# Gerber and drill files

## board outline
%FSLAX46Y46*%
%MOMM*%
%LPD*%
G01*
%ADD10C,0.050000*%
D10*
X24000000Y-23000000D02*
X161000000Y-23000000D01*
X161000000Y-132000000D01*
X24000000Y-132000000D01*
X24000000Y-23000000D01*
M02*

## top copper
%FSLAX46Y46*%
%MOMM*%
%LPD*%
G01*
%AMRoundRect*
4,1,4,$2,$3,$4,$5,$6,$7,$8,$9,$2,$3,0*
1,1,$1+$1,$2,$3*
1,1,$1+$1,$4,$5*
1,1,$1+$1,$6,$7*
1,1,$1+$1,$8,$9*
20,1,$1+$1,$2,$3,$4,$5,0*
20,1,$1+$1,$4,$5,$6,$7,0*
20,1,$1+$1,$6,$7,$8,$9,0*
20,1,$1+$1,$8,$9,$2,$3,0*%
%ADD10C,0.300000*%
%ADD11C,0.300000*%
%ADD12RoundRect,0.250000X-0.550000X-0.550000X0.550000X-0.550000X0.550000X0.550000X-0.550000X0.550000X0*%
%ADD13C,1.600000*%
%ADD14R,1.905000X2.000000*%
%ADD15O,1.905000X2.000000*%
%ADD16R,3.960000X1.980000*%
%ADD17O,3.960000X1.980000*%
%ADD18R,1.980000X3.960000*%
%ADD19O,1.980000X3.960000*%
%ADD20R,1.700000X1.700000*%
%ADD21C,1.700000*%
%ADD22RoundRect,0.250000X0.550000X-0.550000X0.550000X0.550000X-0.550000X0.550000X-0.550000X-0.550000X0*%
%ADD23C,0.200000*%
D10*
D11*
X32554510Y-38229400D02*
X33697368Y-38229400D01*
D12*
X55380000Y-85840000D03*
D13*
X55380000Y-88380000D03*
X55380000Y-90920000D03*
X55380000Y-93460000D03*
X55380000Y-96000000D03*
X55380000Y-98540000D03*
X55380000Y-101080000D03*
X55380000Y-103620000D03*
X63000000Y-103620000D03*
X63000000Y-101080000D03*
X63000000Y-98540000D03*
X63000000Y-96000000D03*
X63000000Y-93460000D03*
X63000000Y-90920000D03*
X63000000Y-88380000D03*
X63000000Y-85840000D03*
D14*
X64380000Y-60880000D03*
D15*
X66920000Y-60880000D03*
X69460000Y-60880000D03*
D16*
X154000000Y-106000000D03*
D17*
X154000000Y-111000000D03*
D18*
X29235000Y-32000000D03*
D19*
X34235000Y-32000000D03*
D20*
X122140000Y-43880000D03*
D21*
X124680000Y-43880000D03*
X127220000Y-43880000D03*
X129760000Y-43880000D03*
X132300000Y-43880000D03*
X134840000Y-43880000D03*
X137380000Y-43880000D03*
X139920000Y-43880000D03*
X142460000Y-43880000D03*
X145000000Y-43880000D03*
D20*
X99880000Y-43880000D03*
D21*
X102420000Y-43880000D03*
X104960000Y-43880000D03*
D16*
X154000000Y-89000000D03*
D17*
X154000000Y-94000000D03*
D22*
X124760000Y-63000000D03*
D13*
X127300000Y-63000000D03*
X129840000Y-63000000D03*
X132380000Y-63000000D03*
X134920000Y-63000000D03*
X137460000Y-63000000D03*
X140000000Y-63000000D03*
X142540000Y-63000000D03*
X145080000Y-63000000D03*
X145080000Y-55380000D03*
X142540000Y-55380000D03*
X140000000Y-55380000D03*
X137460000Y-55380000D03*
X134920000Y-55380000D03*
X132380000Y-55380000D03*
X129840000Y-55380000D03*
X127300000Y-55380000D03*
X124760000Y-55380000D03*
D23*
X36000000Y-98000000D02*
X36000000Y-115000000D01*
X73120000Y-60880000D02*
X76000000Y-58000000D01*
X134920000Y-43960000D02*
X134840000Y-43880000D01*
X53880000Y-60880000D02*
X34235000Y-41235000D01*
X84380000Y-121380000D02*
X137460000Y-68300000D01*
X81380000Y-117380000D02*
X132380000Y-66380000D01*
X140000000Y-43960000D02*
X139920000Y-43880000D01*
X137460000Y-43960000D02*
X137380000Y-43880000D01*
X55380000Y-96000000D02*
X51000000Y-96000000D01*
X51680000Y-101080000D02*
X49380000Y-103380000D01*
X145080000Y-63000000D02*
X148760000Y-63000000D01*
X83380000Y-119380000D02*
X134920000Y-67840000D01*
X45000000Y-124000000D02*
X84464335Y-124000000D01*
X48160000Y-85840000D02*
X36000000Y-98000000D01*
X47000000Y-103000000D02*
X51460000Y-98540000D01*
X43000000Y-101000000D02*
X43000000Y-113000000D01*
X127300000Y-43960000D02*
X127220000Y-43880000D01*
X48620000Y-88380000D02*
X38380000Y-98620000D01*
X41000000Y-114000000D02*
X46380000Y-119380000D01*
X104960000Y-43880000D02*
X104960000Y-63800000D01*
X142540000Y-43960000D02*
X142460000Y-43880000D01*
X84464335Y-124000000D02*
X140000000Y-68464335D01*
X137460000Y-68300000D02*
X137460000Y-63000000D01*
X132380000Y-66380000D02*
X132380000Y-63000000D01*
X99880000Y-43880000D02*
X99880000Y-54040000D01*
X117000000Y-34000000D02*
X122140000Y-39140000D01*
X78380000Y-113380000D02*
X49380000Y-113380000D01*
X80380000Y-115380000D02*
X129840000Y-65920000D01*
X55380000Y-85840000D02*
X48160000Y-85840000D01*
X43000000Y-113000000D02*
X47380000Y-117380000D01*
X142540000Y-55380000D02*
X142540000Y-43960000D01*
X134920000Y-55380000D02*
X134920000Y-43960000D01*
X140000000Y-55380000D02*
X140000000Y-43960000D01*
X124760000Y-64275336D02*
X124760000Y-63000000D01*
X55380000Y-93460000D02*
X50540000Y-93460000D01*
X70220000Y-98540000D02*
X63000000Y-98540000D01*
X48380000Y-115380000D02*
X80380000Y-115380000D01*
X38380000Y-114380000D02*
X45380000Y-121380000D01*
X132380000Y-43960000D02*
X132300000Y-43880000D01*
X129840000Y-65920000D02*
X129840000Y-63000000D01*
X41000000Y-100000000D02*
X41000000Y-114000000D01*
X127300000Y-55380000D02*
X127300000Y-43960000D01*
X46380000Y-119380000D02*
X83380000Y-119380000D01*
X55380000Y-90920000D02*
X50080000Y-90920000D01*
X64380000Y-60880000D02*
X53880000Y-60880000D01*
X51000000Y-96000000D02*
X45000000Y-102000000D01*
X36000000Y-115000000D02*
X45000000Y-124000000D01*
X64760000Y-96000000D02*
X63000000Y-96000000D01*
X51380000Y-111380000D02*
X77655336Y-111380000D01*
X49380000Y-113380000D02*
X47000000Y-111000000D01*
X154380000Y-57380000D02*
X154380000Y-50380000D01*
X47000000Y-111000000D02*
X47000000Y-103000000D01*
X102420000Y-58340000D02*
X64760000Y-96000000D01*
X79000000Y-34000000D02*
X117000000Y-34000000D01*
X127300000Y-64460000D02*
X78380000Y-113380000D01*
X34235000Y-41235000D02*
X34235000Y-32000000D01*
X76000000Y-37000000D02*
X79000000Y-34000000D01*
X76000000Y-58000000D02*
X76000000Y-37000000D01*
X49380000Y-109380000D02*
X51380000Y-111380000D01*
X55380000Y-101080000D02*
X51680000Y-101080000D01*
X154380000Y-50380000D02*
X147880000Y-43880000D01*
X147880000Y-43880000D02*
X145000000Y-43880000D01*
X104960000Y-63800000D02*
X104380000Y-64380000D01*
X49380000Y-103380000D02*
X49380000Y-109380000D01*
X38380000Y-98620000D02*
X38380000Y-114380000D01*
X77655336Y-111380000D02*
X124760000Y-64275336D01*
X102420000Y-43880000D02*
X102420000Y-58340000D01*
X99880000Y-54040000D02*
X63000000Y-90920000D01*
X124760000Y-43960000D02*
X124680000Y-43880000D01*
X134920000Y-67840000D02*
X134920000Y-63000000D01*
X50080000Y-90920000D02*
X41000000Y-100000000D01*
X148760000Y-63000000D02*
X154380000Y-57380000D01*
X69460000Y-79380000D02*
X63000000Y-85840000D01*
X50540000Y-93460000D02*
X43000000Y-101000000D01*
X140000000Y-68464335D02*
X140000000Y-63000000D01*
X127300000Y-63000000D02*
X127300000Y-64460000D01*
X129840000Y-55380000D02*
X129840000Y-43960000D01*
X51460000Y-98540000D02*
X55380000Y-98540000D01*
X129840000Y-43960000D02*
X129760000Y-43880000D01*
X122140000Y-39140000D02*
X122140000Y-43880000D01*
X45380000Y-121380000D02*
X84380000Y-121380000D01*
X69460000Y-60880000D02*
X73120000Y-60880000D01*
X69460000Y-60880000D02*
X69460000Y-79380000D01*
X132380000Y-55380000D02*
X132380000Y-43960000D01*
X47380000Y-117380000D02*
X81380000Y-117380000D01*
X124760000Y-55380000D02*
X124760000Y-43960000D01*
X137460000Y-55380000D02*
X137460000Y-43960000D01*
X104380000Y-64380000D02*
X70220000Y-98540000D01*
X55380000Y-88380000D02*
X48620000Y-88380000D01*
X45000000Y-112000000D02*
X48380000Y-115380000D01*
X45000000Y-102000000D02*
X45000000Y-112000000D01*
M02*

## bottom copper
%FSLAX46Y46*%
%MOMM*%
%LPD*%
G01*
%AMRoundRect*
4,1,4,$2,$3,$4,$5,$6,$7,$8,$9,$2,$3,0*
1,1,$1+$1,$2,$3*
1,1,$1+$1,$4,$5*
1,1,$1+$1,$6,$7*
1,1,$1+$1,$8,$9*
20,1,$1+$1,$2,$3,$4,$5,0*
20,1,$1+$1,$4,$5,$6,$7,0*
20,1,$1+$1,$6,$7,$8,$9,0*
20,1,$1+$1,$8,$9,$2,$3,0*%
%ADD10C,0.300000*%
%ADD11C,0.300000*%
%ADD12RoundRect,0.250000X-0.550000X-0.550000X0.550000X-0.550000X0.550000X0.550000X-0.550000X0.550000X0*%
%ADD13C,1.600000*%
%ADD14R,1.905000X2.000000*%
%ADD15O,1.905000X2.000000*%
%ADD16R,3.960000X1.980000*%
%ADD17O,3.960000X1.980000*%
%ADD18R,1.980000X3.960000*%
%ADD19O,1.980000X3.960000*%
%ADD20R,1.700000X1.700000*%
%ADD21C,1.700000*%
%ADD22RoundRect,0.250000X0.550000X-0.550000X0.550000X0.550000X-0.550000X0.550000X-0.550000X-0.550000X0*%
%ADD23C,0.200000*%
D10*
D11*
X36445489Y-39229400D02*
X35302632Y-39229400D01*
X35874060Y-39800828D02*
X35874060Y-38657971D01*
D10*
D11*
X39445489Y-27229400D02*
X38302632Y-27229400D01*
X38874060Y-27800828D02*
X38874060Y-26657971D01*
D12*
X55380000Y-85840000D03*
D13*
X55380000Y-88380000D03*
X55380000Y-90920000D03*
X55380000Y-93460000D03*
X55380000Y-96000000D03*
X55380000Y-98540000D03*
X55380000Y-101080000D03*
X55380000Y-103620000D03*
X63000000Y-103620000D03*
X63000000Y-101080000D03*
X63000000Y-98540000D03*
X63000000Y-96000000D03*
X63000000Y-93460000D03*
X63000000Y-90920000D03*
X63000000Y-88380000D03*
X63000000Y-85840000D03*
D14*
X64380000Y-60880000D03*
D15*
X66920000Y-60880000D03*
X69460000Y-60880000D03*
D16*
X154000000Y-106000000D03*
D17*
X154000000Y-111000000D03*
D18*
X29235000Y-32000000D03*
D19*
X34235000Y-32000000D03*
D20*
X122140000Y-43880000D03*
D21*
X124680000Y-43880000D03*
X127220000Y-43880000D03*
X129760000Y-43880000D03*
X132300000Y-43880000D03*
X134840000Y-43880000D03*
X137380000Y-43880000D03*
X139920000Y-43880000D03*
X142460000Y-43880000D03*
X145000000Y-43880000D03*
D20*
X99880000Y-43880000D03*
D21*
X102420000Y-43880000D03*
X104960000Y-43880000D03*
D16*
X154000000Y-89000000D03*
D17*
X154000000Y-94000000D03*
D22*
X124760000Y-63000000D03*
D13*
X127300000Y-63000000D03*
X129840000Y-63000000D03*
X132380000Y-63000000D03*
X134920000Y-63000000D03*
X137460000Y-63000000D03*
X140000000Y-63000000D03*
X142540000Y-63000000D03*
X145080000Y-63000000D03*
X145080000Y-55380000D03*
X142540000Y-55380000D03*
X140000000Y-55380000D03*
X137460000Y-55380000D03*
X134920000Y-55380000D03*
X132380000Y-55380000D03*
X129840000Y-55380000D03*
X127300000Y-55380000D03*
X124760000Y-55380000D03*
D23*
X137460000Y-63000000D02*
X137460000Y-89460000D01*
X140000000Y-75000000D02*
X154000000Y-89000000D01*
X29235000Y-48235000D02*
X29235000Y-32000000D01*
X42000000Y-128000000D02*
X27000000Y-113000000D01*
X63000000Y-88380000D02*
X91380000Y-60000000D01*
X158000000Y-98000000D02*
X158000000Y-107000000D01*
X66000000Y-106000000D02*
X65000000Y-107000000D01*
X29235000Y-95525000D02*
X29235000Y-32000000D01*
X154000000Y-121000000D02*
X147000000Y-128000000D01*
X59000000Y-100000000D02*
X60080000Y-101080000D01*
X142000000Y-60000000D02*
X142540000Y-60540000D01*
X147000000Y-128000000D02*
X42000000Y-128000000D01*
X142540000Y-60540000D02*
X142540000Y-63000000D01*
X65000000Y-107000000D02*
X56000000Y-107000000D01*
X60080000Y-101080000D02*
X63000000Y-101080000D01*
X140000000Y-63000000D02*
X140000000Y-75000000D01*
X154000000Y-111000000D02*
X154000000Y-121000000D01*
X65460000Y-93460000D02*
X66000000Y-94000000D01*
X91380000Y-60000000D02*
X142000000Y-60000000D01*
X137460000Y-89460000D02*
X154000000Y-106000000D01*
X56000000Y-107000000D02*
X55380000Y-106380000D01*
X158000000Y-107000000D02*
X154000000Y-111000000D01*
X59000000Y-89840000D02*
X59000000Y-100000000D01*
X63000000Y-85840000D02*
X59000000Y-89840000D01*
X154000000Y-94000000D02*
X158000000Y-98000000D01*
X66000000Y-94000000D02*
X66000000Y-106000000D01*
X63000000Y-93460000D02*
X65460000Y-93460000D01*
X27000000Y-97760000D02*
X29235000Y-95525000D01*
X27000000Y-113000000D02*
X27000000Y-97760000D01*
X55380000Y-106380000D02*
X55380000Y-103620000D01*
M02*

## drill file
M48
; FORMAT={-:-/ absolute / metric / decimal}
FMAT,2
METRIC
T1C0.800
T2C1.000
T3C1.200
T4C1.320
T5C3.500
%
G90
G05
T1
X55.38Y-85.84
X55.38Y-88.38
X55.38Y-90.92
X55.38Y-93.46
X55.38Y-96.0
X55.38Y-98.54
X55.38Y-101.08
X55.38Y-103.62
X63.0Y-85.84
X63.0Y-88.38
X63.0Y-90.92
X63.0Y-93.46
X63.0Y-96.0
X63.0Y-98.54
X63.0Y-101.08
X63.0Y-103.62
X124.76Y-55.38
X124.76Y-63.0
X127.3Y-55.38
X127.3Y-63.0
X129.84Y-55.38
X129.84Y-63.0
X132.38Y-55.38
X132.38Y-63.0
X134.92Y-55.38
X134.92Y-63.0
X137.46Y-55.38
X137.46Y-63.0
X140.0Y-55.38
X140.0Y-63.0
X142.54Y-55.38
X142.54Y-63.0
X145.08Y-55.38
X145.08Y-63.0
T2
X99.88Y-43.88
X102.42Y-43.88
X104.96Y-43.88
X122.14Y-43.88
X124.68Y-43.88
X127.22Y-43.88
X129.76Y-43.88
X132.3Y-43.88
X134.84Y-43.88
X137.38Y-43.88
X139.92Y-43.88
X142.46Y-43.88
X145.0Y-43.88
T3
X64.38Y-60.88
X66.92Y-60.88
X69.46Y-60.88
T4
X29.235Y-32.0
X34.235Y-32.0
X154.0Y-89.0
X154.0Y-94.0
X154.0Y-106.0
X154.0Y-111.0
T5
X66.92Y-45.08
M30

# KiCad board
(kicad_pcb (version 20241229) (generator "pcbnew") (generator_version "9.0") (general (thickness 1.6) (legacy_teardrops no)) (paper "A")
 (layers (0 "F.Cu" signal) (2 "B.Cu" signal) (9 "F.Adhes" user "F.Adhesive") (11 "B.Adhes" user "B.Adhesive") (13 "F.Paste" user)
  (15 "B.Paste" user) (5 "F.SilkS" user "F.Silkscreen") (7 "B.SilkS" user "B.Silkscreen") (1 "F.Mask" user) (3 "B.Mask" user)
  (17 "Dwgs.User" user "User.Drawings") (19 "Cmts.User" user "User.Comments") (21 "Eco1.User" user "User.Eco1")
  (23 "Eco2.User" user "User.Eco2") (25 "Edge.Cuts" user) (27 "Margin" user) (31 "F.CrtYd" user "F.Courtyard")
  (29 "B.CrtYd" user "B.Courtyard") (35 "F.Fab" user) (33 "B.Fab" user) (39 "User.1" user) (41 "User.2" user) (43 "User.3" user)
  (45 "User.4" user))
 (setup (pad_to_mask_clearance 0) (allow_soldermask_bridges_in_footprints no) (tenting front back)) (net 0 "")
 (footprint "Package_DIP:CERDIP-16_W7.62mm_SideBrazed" (layer "F.Cu") (at 55.38 85.84)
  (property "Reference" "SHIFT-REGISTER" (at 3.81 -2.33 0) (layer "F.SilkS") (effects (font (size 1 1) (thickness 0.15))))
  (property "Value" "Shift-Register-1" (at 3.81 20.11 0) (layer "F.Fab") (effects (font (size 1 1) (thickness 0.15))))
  (pad "1" thru_hole roundrect (at 0 0) (size 1.6 1.6) (drill 0.8) (layers "*.Cu" "*.Mask") (remove_unused_layers no)
   (roundrect_rratio 0.15625))
  (pad "2" thru_hole circle (at 0 2.54) (size 1.6 1.6) (drill 0.8) (layers "*.Cu" "*.Mask") (remove_unused_layers no))
  (pad "3" thru_hole circle (at 0 5.08) (size 1.6 1.6) (drill 0.8) (layers "*.Cu" "*.Mask") (remove_unused_layers no))
  (pad "4" thru_hole circle (at 0 7.62) (size 1.6 1.6) (drill 0.8) (layers "*.Cu" "*.Mask") (remove_unused_layers no))
  (pad "5" thru_hole circle (at 0 10.16) (size 1.6 1.6) (drill 0.8) (layers "*.Cu" "*.Mask") (remove_unused_layers no))
  (pad "6" thru_hole circle (at 0 12.7) (size 1.6 1.6) (drill 0.8) (layers "*.Cu" "*.Mask") (remove_unused_layers no))
  (pad "7" thru_hole circle (at 0 15.24) (size 1.6 1.6) (drill 0.8) (layers "*.Cu" "*.Mask") (remove_unused_layers no))
  (pad "8" thru_hole circle (at 0 17.78) (size 1.6 1.6) (drill 0.8) (layers "*.Cu" "*.Mask") (remove_unused_layers no))
  (pad "9" thru_hole circle (at 7.62 17.78) (size 1.6 1.6) (drill 0.8) (layers "*.Cu" "*.Mask") (remove_unused_layers no))
  (pad "10" thru_hole circle (at 7.62 15.24) (size 1.6 1.6) (drill 0.8) (layers "*.Cu" "*.Mask") (remove_unused_layers no))
  (pad "11" thru_hole circle (at 7.62 12.7) (size 1.6 1.6) (drill 0.8) (layers "*.Cu" "*.Mask") (remove_unused_layers no))
  (pad "12" thru_hole circle (at 7.62 10.16) (size 1.6 1.6) (drill 0.8) (layers "*.Cu" "*.Mask") (remove_unused_layers no))
  (pad "13" thru_hole circle (at 7.62 7.62) (size 1.6 1.6) (drill 0.8) (layers "*.Cu" "*.Mask") (remove_unused_layers no))
  (pad "14" thru_hole circle (at 7.62 5.08) (size 1.6 1.6) (drill 0.8) (layers "*.Cu" "*.Mask") (remove_unused_layers no))
  (pad "15" thru_hole circle (at 7.62 2.54) (size 1.6 1.6) (drill 0.8) (layers "*.Cu" "*.Mask") (remove_unused_layers no))
  (pad "16" thru_hole circle (at 7.62 0) (size 1.6 1.6) (drill 0.8) (layers "*.Cu" "*.Mask") (remove_unused_layers no)))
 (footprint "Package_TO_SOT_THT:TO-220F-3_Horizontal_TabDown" (layer "F.Cu") (at 64.38 60.88)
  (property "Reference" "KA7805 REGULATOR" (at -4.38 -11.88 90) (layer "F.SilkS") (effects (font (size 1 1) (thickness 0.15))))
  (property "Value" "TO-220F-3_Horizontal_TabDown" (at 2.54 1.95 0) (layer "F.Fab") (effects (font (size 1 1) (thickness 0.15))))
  (pad "" np_thru_hole circle (at 2.54 -15.8) (size 3.5 3.5) (drill 3.5) (layers "*.Cu" "*.Mask"))
  (pad "1" thru_hole rect (at 0 0) (size 1.905 2) (drill 1.2) (layers "*.Cu" "*.Mask") (remove_unused_layers no))
  (pad "2" thru_hole oval (at 2.54 0) (size 1.905 2) (drill 1.2) (layers "*.Cu" "*.Mask") (remove_unused_layers no))
  (pad "3" thru_hole oval (at 5.08 0) (size 1.905 2) (drill 1.2) (layers "*.Cu" "*.Mask") (remove_unused_layers no)))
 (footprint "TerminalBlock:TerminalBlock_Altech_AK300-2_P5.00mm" (layer "F.Cu") (at 154 106 -90)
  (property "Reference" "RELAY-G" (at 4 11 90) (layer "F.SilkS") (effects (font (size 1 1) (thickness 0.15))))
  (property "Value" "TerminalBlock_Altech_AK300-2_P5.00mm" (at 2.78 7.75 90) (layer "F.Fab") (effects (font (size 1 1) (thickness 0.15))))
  (pad "1" thru_hole rect (at 0 0 270) (size 1.98 3.96) (drill 1.32) (layers "*.Cu" "*.Mask") (remove_unused_layers no))
  (pad "2" thru_hole oval (at 5 0 270) (size 1.98 3.96) (drill 1.32) (layers "*.Cu" "*.Mask") (remove_unused_layers no)))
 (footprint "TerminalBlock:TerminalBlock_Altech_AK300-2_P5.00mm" (layer "F.Cu") (at 29.235 32)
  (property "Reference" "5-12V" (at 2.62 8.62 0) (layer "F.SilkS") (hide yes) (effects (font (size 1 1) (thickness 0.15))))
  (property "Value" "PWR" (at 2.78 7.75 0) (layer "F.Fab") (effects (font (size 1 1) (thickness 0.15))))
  (pad "1" thru_hole rect (at 0 0) (size 1.98 3.96) (drill 1.32) (layers "*.Cu" "*.Mask") (remove_unused_layers no))
  (pad "2" thru_hole oval (at 5 0) (size 1.98 3.96) (drill 1.32) (layers "*.Cu" "*.Mask") (remove_unused_layers no)))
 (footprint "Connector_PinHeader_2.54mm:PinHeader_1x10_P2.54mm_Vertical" (layer "F.Cu") (at 122.14 43.88 90)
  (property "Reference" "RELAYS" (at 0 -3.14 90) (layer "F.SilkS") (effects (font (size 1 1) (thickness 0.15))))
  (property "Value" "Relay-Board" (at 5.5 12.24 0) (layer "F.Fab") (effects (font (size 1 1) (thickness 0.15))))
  (pad "1" thru_hole rect (at 0 0 90) (size 1.7 1.7) (drill 1) (layers "*.Cu" "*.Mask") (remove_unused_layers no))
  (pad "2" thru_hole circle (at 0 2.54 90) (size 1.7 1.7) (drill 1) (layers "*.Cu" "*.Mask") (remove_unused_layers no))
  (pad "3" thru_hole circle (at 0 5.08 90) (size 1.7 1.7) (drill 1) (layers "*.Cu" "*.Mask") (remove_unused_layers no))
  (pad "4" thru_hole circle (at 0 7.62 90) (size 1.7 1.7) (drill 1) (layers "*.Cu" "*.Mask") (remove_unused_layers no))
  (pad "5" thru_hole circle (at 0 10.16 90) (size 1.7 1.7) (drill 1) (layers "*.Cu" "*.Mask") (remove_unused_layers no))
  (pad "6" thru_hole circle (at 0 12.7 90) (size 1.7 1.7) (drill 1) (layers "*.Cu" "*.Mask") (remove_unused_layers no))
  (pad "7" thru_hole circle (at 0 15.24 90) (size 1.7 1.7) (drill 1) (layers "*.Cu" "*.Mask") (remove_unused_layers no))
  (pad "8" thru_hole circle (at 0 17.78 90) (size 1.7 1.7) (drill 1) (layers "*.Cu" "*.Mask") (remove_unused_layers no))
  (pad "9" thru_hole circle (at 0 20.32 90) (size 1.7 1.7) (drill 1) (layers "*.Cu" "*.Mask") (remove_unused_layers no))
  (pad "10" thru_hole circle (at 0 22.86 90) (size 1.7 1.7) (drill 1) (layers "*.Cu" "*.Mask") (remove_unused_layers no)))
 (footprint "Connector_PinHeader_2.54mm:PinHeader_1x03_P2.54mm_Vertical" (layer "F.Cu") (at 99.88 43.88 90)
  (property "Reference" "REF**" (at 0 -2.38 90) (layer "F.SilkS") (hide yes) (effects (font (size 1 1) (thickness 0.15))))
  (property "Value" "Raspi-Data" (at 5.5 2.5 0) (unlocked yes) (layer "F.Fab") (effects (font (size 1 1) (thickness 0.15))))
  (pad "1" thru_hole rect (at 0 0 90) (size 1.7 1.7) (drill 1) (layers "*.Cu" "*.Mask") (remove_unused_layers no))
  (pad "2" thru_hole circle (at 0 2.54 90) (size 1.7 1.7) (drill 1) (layers "*.Cu" "*.Mask") (remove_unused_layers no))
  (pad "3" thru_hole circle (at 0 5.08 90) (size 1.7 1.7) (drill 1) (layers "*.Cu" "*.Mask") (remove_unused_layers no)))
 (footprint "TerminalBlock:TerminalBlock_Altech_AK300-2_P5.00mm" (layer "F.Cu") (at 154 89 -90)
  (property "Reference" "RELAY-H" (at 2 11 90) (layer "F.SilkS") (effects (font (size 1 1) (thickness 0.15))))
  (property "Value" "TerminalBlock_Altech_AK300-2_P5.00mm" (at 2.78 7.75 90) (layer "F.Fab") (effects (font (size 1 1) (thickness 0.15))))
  (pad "1" thru_hole rect (at 0 0 270) (size 1.98 3.96) (drill 1.32) (layers "*.Cu" "*.Mask") (remove_unused_layers no))
  (pad "2" thru_hole oval (at 5 0 270) (size 1.98 3.96) (drill 1.32) (layers "*.Cu" "*.Mask") (remove_unused_layers no)))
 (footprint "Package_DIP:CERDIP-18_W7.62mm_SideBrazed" (layer "F.Cu") (at 124.76 63 90)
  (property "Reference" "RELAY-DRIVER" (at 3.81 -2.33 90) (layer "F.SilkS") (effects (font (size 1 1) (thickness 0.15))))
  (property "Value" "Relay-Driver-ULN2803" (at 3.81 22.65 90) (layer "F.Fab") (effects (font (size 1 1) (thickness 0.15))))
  (pad "1" thru_hole roundrect (at 0 0 90) (size 1.6 1.6) (drill 0.8) (layers "*.Cu" "*.Mask") (remove_unused_layers no)
   (roundrect_rratio 0.15625))
  (pad "2" thru_hole circle (at 0 2.54 90) (size 1.6 1.6) (drill 0.8) (layers "*.Cu" "*.Mask") (remove_unused_layers no))
  (pad "3" thru_hole circle (at 0 5.08 90) (size 1.6 1.6) (drill 0.8) (layers "*.Cu" "*.Mask") (remove_unused_layers no))
  (pad "4" thru_hole circle (at 0 7.62 90) (size 1.6 1.6) (drill 0.8) (layers "*.Cu" "*.Mask") (remove_unused_layers no))
  (pad "5" thru_hole circle (at 0 10.16 90) (size 1.6 1.6) (drill 0.8) (layers "*.Cu" "*.Mask") (remove_unused_layers no))
  (pad "6" thru_hole circle (at 0 12.7 90) (size 1.6 1.6) (drill 0.8) (layers "*.Cu" "*.Mask") (remove_unused_layers no))
  (pad "7" thru_hole circle (at 0 15.24 90) (size 1.6 1.6) (drill 0.8) (layers "*.Cu" "*.Mask") (remove_unused_layers no))
  (pad "8" thru_hole circle (at 0 17.78 90) (size 1.6 1.6) (drill 0.8) (layers "*.Cu" "*.Mask") (remove_unused_layers no))
  (pad "9" thru_hole circle (at 0 20.32 90) (size 1.6 1.6) (drill 0.8) (layers "*.Cu" "*.Mask") (remove_unused_layers no))
  (pad "10" thru_hole circle (at 7.62 20.32 90) (size 1.6 1.6) (drill 0.8) (layers "*.Cu" "*.Mask") (remove_unused_layers no))
  (pad "11" thru_hole circle (at 7.62 17.78 90) (size 1.6 1.6) (drill 0.8) (layers "*.Cu" "*.Mask") (remove_unused_layers no))
  (pad "12" thru_hole circle (at 7.62 15.24 90) (size 1.6 1.6) (drill 0.8) (layers "*.Cu" "*.Mask") (remove_unused_layers no))
  (pad "13" thru_hole circle (at 7.62 12.7 90) (size 1.6 1.6) (drill 0.8) (layers "*.Cu" "*.Mask") (remove_unused_layers no))
  (pad "14" thru_hole circle (at 7.62 10.16 90) (size 1.6 1.6) (drill 0.8) (layers "*.Cu" "*.Mask") (remove_unused_layers no))
  (pad "15" thru_hole circle (at 7.62 7.62 90) (size 1.6 1.6) (drill 0.8) (layers "*.Cu" "*.Mask") (remove_unused_layers no))
  (pad "16" thru_hole circle (at 7.62 5.08 90) (size 1.6 1.6) (drill 0.8) (layers "*.Cu" "*.Mask") (remove_unused_layers no))
  (pad "17" thru_hole circle (at 7.62 2.54 90) (size 1.6 1.6) (drill 0.8) (layers "*.Cu" "*.Mask") (remove_unused_layers no))
  (pad "18" thru_hole circle (at 7.62 0 90) (size 1.6 1.6) (drill 0.8) (layers "*.Cu" "*.Mask") (remove_unused_layers no)))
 (gr_rect (start 24 23) (end 161 132) (stroke (width 0.05) (type default)) (fill no) (layer "Edge.Cuts"))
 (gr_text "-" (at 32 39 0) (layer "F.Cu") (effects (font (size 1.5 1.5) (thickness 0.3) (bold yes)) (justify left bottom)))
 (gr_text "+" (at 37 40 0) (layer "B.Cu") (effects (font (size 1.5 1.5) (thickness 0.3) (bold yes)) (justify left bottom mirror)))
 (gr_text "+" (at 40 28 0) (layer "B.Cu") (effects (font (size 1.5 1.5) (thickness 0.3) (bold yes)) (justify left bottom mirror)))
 (segment (start 36 98) (end 36 115) (width 0.2) (layer "F.Cu") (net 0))
 (segment (start 73.12 60.88) (end 76 58) (width 0.2) (layer "F.Cu") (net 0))
 (segment (start 134.92 43.96) (end 134.84 43.88) (width 0.2) (layer "F.Cu") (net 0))
 (segment (start 53.88 60.88) (end 34.235 41.235) (width 0.2) (layer "F.Cu") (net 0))
 (segment (start 84.38 121.38) (end 137.46 68.3) (width 0.2) (layer "F.Cu") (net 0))
 (segment (start 81.38 117.38) (end 132.38 66.38) (width 0.2) (layer "F.Cu") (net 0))
 (segment (start 140 43.96) (end 139.92 43.88) (width 0.2) (layer "F.Cu") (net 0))
 (segment (start 137.46 43.96) (end 137.38 43.88) (width 0.2) (layer "F.Cu") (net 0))
 (segment (start 55.38 96) (end 51 96) (width 0.2) (layer "F.Cu") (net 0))
 (segment (start 51.68 101.08) (end 49.38 103.38) (width 0.2) (layer "F.Cu") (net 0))
 (segment (start 145.08 63) (end 148.76 63) (width 0.2) (layer "F.Cu") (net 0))
 (segment (start 83.38 119.38) (end 134.92 67.84) (width 0.2) (layer "F.Cu") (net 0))
 (segment (start 45 124) (end 84.464335 124) (width 0.2) (layer "F.Cu") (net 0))
 (segment (start 48.16 85.84) (end 36 98) (width 0.2) (layer "F.Cu") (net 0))
 (segment (start 47 103) (end 51.46 98.54) (width 0.2) (layer "F.Cu") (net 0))
 (segment (start 43 101) (end 43 113) (width 0.2) (layer "F.Cu") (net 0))
 (segment (start 127.3 43.96) (end 127.22 43.88) (width 0.2) (layer "F.Cu") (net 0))
 (segment (start 48.62 88.38) (end 38.38 98.62) (width 0.2) (layer "F.Cu") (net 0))
 (segment (start 41 114) (end 46.38 119.38) (width 0.2) (layer "F.Cu") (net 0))
 (segment (start 104.96 43.88) (end 104.96 63.8) (width 0.2) (layer "F.Cu") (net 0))
 (segment (start 142.54 43.96) (end 142.46 43.88) (width 0.2) (layer "F.Cu") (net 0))
 (segment (start 84.464335 124) (end 140 68.464335) (width 0.2) (layer "F.Cu") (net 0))
 (segment (start 137.46 68.3) (end 137.46 63) (width 0.2) (layer "F.Cu") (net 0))
 (segment (start 132.38 66.38) (end 132.38 63) (width 0.2) (layer "F.Cu") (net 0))
 (segment (start 99.88 43.88) (end 99.88 54.04) (width 0.2) (layer "F.Cu") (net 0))
 (segment (start 117 34) (end 122.14 39.14) (width 0.2) (layer "F.Cu") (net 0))
 (segment (start 78.38 113.38) (end 49.38 113.38) (width 0.2) (layer "F.Cu") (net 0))
 (segment (start 80.38 115.38) (end 129.84 65.92) (width 0.2) (layer "F.Cu") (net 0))
 (segment (start 55.38 85.84) (end 48.16 85.84) (width 0.2) (layer "F.Cu") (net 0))
 (segment (start 43 113) (end 47.38 117.38) (width 0.2) (layer "F.Cu") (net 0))
 (segment (start 142.54 55.38) (end 142.54 43.96) (width 0.2) (layer "F.Cu") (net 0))
 (segment (start 134.92 55.38) (end 134.92 43.96) (width 0.2) (layer "F.Cu") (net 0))
 (segment (start 140 55.38) (end 140 43.96) (width 0.2) (layer "F.Cu") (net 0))
 (segment (start 124.76 64.275336) (end 124.76 63) (width 0.2) (layer "F.Cu") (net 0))
 (segment (start 55.38 93.46) (end 50.54 93.46) (width 0.2) (layer "F.Cu") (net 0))
 (segment (start 70.22 98.54) (end 63 98.54) (width 0.2) (layer "F.Cu") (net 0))
 (segment (start 48.38 115.38) (end 80.38 115.38) (width 0.2) (layer "F.Cu") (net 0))
 (segment (start 38.38 114.38) (end 45.38 121.38) (width 0.2) (layer "F.Cu") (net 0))
 (segment (start 132.38 43.96) (end 132.3 43.88) (width 0.2) (layer "F.Cu") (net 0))
 (segment (start 129.84 65.92) (end 129.84 63) (width 0.2) (layer "F.Cu") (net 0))
 (segment (start 41 100) (end 41 114) (width 0.2) (layer "F.Cu") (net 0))
 (segment (start 127.3 55.38) (end 127.3 43.96) (width 0.2) (layer "F.Cu") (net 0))
 (segment (start 46.38 119.38) (end 83.38 119.38) (width 0.2) (layer "F.Cu") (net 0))
 (segment (start 55.38 90.92) (end 50.08 90.92) (width 0.2) (layer "F.Cu") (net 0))
 (segment (start 64.38 60.88) (end 53.88 60.88) (width 0.2) (layer "F.Cu") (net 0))
 (segment (start 51 96) (end 45 102) (width 0.2) (layer "F.Cu") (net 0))
 (segment (start 36 115) (end 45 124) (width 0.2) (layer "F.Cu") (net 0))
 (segment (start 64.76 96) (end 63 96) (width 0.2) (layer "F.Cu") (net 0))
 (segment (start 51.38 111.38) (end 77.655336 111.38) (width 0.2) (layer "F.Cu") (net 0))
 (segment (start 49.38 113.38) (end 47 111) (width 0.2) (layer "F.Cu") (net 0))
 (segment (start 154.38 57.38) (end 154.38 50.38) (width 0.2) (layer "F.Cu") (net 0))
 (segment (start 47 111) (end 47 103) (width 0.2) (layer "F.Cu") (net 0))
 (segment (start 102.42 58.34) (end 64.76 96) (width 0.2) (layer "F.Cu") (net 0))
 (segment (start 79 34) (end 117 34) (width 0.2) (layer "F.Cu") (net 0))
 (segment (start 127.3 64.46) (end 78.38 113.38) (width 0.2) (layer "F.Cu") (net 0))
 (segment (start 34.235 41.235) (end 34.235 32) (width 0.2) (layer "F.Cu") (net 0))
 (segment (start 76 37) (end 79 34) (width 0.2) (layer "F.Cu") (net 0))
 (segment (start 76 58) (end 76 37) (width 0.2) (layer "F.Cu") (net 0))
 (segment (start 49.38 109.38) (end 51.38 111.38) (width 0.2) (layer "F.Cu") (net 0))
 (segment (start 55.38 101.08) (end 51.68 101.08) (width 0.2) (layer "F.Cu") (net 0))
 (segment (start 154.38 50.38) (end 147.88 43.88) (width 0.2) (layer "F.Cu") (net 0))
 (segment (start 147.88 43.88) (end 145 43.88) (width 0.2) (layer "F.Cu") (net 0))
 (segment (start 104.96 63.8) (end 104.38 64.38) (width 0.2) (layer "F.Cu") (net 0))
 (segment (start 49.38 103.38) (end 49.38 109.38) (width 0.2) (layer "F.Cu") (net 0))
 (segment (start 38.38 98.62) (end 38.38 114.38) (width 0.2) (layer "F.Cu") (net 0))
 (segment (start 77.655336 111.38) (end 124.76 64.275336) (width 0.2) (layer "F.Cu") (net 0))
 (segment (start 102.42 43.88) (end 102.42 58.34) (width 0.2) (layer "F.Cu") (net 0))
 (segment (start 99.88 54.04) (end 63 90.92) (width 0.2) (layer "F.Cu") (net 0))
 (segment (start 124.76 43.96) (end 124.68 43.88) (width 0.2) (layer "F.Cu") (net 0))
 (segment (start 134.92 67.84) (end 134.92 63) (width 0.2) (layer "F.Cu") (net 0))
 (segment (start 50.08 90.92) (end 41 100) (width 0.2) (layer "F.Cu") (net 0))
 (segment (start 148.76 63) (end 154.38 57.38) (width 0.2) (layer "F.Cu") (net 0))
 (segment (start 69.46 79.38) (end 63 85.84) (width 0.2) (layer "F.Cu") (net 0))
 (segment (start 50.54 93.46) (end 43 101) (width 0.2) (layer "F.Cu") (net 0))
 (segment (start 140 68.464335) (end 140 63) (width 0.2) (layer "F.Cu") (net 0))
 (segment (start 127.3 63) (end 127.3 64.46) (width 0.2) (layer "F.Cu") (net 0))
 (segment (start 129.84 55.38) (end 129.84 43.96) (width 0.2) (layer "F.Cu") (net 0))
 (segment (start 51.46 98.54) (end 55.38 98.54) (width 0.2) (layer "F.Cu") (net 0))
 (segment (start 129.84 43.96) (end 129.76 43.88) (width 0.2) (layer "F.Cu") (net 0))
 (segment (start 122.14 39.14) (end 122.14 43.88) (width 0.2) (layer "F.Cu") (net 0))
 (segment (start 45.38 121.38) (end 84.38 121.38) (width 0.2) (layer "F.Cu") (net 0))
 (segment (start 69.46 60.88) (end 73.12 60.88) (width 0.2) (layer "F.Cu") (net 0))
 (segment (start 69.46 60.88) (end 69.46 79.38) (width 0.2) (layer "F.Cu") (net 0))
 (segment (start 132.38 55.38) (end 132.38 43.96) (width 0.2) (layer "F.Cu") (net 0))
 (segment (start 47.38 117.38) (end 81.38 117.38) (width 0.2) (layer "F.Cu") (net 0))
 (segment (start 124.76 55.38) (end 124.76 43.96) (width 0.2) (layer "F.Cu") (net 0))
 (segment (start 137.46 55.38) (end 137.46 43.96) (width 0.2) (layer "F.Cu") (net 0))
 (segment (start 104.38 64.38) (end 70.22 98.54) (width 0.2) (layer "F.Cu") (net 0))
 (segment (start 55.38 88.38) (end 48.62 88.38) (width 0.2) (layer "F.Cu") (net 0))
 (segment (start 45 112) (end 48.38 115.38) (width 0.2) (layer "F.Cu") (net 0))
 (segment (start 45 102) (end 45 112) (width 0.2) (layer "F.Cu") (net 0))
 (segment (start 137.46 63) (end 137.46 89.46) (width 0.2) (layer "B.Cu") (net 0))
 (segment (start 140 75) (end 154 89) (width 0.2) (layer "B.Cu") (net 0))
 (segment (start 29.235 48.235) (end 29.235 32) (width 0.2) (layer "B.Cu") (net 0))
 (segment (start 42 128) (end 27 113) (width 0.2) (layer "B.Cu") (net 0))
 (segment (start 63 88.38) (end 91.38 60) (width 0.2) (layer "B.Cu") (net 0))
 (segment (start 158 98) (end 158 107) (width 0.2) (layer "B.Cu") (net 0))
 (segment (start 66 106) (end 65 107) (width 0.2) (layer "B.Cu") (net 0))
 (segment (start 29.235 95.525) (end 29.235 32) (width 0.2) (layer "B.Cu") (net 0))
 (segment (start 154 121) (end 147 128) (width 0.2) (layer "B.Cu") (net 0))
 (segment (start 59 100) (end 60.08 101.08) (width 0.2) (layer "B.Cu") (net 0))
 (segment (start 142 60) (end 142.54 60.54) (width 0.2) (layer "B.Cu") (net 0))
 (segment (start 147 128) (end 42 128) (width 0.2) (layer "B.Cu") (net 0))
 (segment (start 142.54 60.54) (end 142.54 63) (width 0.2) (layer "B.Cu") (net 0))
 (segment (start 65 107) (end 56 107) (width 0.2) (layer "B.Cu") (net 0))
 (segment (start 60.08 101.08) (end 63 101.08) (width 0.2) (layer "B.Cu") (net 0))
 (segment (start 140 63) (end 140 75) (width 0.2) (layer "B.Cu") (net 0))
 (segment (start 154 111) (end 154 121) (width 0.2) (layer "B.Cu") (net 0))
 (segment (start 65.46 93.46) (end 66 94) (width 0.2) (layer "B.Cu") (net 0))
 (segment (start 91.38 60) (end 142 60) (width 0.2) (layer "B.Cu") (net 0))
 (segment (start 137.46 89.46) (end 154 106) (width 0.2) (layer "B.Cu") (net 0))
 (segment (start 56 107) (end 55.38 106.38) (width 0.2) (layer "B.Cu") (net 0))
 (segment (start 158 107) (end 154 111) (width 0.2) (layer "B.Cu") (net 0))
 (segment (start 59 89.84) (end 59 100) (width 0.2) (layer "B.Cu") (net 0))
 (segment (start 63 85.84) (end 59 89.84) (width 0.2) (layer "B.Cu") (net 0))
 (segment (start 154 94) (end 158 98) (width 0.2) (layer "B.Cu") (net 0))
 (segment (start 66 94) (end 66 106) (width 0.2) (layer "B.Cu") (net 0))
 (segment (start 63 93.46) (end 65.46 93.46) (width 0.2) (layer "B.Cu") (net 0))
 (segment (start 27 97.76) (end 29.235 95.525) (width 0.2) (layer "B.Cu") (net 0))
 (segment (start 27 113) (end 27 97.76) (width 0.2) (layer "B.Cu") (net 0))
 (segment (start 55.38 106.38) (end 55.38 103.62) (width 0.2) (layer "B.Cu") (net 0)))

